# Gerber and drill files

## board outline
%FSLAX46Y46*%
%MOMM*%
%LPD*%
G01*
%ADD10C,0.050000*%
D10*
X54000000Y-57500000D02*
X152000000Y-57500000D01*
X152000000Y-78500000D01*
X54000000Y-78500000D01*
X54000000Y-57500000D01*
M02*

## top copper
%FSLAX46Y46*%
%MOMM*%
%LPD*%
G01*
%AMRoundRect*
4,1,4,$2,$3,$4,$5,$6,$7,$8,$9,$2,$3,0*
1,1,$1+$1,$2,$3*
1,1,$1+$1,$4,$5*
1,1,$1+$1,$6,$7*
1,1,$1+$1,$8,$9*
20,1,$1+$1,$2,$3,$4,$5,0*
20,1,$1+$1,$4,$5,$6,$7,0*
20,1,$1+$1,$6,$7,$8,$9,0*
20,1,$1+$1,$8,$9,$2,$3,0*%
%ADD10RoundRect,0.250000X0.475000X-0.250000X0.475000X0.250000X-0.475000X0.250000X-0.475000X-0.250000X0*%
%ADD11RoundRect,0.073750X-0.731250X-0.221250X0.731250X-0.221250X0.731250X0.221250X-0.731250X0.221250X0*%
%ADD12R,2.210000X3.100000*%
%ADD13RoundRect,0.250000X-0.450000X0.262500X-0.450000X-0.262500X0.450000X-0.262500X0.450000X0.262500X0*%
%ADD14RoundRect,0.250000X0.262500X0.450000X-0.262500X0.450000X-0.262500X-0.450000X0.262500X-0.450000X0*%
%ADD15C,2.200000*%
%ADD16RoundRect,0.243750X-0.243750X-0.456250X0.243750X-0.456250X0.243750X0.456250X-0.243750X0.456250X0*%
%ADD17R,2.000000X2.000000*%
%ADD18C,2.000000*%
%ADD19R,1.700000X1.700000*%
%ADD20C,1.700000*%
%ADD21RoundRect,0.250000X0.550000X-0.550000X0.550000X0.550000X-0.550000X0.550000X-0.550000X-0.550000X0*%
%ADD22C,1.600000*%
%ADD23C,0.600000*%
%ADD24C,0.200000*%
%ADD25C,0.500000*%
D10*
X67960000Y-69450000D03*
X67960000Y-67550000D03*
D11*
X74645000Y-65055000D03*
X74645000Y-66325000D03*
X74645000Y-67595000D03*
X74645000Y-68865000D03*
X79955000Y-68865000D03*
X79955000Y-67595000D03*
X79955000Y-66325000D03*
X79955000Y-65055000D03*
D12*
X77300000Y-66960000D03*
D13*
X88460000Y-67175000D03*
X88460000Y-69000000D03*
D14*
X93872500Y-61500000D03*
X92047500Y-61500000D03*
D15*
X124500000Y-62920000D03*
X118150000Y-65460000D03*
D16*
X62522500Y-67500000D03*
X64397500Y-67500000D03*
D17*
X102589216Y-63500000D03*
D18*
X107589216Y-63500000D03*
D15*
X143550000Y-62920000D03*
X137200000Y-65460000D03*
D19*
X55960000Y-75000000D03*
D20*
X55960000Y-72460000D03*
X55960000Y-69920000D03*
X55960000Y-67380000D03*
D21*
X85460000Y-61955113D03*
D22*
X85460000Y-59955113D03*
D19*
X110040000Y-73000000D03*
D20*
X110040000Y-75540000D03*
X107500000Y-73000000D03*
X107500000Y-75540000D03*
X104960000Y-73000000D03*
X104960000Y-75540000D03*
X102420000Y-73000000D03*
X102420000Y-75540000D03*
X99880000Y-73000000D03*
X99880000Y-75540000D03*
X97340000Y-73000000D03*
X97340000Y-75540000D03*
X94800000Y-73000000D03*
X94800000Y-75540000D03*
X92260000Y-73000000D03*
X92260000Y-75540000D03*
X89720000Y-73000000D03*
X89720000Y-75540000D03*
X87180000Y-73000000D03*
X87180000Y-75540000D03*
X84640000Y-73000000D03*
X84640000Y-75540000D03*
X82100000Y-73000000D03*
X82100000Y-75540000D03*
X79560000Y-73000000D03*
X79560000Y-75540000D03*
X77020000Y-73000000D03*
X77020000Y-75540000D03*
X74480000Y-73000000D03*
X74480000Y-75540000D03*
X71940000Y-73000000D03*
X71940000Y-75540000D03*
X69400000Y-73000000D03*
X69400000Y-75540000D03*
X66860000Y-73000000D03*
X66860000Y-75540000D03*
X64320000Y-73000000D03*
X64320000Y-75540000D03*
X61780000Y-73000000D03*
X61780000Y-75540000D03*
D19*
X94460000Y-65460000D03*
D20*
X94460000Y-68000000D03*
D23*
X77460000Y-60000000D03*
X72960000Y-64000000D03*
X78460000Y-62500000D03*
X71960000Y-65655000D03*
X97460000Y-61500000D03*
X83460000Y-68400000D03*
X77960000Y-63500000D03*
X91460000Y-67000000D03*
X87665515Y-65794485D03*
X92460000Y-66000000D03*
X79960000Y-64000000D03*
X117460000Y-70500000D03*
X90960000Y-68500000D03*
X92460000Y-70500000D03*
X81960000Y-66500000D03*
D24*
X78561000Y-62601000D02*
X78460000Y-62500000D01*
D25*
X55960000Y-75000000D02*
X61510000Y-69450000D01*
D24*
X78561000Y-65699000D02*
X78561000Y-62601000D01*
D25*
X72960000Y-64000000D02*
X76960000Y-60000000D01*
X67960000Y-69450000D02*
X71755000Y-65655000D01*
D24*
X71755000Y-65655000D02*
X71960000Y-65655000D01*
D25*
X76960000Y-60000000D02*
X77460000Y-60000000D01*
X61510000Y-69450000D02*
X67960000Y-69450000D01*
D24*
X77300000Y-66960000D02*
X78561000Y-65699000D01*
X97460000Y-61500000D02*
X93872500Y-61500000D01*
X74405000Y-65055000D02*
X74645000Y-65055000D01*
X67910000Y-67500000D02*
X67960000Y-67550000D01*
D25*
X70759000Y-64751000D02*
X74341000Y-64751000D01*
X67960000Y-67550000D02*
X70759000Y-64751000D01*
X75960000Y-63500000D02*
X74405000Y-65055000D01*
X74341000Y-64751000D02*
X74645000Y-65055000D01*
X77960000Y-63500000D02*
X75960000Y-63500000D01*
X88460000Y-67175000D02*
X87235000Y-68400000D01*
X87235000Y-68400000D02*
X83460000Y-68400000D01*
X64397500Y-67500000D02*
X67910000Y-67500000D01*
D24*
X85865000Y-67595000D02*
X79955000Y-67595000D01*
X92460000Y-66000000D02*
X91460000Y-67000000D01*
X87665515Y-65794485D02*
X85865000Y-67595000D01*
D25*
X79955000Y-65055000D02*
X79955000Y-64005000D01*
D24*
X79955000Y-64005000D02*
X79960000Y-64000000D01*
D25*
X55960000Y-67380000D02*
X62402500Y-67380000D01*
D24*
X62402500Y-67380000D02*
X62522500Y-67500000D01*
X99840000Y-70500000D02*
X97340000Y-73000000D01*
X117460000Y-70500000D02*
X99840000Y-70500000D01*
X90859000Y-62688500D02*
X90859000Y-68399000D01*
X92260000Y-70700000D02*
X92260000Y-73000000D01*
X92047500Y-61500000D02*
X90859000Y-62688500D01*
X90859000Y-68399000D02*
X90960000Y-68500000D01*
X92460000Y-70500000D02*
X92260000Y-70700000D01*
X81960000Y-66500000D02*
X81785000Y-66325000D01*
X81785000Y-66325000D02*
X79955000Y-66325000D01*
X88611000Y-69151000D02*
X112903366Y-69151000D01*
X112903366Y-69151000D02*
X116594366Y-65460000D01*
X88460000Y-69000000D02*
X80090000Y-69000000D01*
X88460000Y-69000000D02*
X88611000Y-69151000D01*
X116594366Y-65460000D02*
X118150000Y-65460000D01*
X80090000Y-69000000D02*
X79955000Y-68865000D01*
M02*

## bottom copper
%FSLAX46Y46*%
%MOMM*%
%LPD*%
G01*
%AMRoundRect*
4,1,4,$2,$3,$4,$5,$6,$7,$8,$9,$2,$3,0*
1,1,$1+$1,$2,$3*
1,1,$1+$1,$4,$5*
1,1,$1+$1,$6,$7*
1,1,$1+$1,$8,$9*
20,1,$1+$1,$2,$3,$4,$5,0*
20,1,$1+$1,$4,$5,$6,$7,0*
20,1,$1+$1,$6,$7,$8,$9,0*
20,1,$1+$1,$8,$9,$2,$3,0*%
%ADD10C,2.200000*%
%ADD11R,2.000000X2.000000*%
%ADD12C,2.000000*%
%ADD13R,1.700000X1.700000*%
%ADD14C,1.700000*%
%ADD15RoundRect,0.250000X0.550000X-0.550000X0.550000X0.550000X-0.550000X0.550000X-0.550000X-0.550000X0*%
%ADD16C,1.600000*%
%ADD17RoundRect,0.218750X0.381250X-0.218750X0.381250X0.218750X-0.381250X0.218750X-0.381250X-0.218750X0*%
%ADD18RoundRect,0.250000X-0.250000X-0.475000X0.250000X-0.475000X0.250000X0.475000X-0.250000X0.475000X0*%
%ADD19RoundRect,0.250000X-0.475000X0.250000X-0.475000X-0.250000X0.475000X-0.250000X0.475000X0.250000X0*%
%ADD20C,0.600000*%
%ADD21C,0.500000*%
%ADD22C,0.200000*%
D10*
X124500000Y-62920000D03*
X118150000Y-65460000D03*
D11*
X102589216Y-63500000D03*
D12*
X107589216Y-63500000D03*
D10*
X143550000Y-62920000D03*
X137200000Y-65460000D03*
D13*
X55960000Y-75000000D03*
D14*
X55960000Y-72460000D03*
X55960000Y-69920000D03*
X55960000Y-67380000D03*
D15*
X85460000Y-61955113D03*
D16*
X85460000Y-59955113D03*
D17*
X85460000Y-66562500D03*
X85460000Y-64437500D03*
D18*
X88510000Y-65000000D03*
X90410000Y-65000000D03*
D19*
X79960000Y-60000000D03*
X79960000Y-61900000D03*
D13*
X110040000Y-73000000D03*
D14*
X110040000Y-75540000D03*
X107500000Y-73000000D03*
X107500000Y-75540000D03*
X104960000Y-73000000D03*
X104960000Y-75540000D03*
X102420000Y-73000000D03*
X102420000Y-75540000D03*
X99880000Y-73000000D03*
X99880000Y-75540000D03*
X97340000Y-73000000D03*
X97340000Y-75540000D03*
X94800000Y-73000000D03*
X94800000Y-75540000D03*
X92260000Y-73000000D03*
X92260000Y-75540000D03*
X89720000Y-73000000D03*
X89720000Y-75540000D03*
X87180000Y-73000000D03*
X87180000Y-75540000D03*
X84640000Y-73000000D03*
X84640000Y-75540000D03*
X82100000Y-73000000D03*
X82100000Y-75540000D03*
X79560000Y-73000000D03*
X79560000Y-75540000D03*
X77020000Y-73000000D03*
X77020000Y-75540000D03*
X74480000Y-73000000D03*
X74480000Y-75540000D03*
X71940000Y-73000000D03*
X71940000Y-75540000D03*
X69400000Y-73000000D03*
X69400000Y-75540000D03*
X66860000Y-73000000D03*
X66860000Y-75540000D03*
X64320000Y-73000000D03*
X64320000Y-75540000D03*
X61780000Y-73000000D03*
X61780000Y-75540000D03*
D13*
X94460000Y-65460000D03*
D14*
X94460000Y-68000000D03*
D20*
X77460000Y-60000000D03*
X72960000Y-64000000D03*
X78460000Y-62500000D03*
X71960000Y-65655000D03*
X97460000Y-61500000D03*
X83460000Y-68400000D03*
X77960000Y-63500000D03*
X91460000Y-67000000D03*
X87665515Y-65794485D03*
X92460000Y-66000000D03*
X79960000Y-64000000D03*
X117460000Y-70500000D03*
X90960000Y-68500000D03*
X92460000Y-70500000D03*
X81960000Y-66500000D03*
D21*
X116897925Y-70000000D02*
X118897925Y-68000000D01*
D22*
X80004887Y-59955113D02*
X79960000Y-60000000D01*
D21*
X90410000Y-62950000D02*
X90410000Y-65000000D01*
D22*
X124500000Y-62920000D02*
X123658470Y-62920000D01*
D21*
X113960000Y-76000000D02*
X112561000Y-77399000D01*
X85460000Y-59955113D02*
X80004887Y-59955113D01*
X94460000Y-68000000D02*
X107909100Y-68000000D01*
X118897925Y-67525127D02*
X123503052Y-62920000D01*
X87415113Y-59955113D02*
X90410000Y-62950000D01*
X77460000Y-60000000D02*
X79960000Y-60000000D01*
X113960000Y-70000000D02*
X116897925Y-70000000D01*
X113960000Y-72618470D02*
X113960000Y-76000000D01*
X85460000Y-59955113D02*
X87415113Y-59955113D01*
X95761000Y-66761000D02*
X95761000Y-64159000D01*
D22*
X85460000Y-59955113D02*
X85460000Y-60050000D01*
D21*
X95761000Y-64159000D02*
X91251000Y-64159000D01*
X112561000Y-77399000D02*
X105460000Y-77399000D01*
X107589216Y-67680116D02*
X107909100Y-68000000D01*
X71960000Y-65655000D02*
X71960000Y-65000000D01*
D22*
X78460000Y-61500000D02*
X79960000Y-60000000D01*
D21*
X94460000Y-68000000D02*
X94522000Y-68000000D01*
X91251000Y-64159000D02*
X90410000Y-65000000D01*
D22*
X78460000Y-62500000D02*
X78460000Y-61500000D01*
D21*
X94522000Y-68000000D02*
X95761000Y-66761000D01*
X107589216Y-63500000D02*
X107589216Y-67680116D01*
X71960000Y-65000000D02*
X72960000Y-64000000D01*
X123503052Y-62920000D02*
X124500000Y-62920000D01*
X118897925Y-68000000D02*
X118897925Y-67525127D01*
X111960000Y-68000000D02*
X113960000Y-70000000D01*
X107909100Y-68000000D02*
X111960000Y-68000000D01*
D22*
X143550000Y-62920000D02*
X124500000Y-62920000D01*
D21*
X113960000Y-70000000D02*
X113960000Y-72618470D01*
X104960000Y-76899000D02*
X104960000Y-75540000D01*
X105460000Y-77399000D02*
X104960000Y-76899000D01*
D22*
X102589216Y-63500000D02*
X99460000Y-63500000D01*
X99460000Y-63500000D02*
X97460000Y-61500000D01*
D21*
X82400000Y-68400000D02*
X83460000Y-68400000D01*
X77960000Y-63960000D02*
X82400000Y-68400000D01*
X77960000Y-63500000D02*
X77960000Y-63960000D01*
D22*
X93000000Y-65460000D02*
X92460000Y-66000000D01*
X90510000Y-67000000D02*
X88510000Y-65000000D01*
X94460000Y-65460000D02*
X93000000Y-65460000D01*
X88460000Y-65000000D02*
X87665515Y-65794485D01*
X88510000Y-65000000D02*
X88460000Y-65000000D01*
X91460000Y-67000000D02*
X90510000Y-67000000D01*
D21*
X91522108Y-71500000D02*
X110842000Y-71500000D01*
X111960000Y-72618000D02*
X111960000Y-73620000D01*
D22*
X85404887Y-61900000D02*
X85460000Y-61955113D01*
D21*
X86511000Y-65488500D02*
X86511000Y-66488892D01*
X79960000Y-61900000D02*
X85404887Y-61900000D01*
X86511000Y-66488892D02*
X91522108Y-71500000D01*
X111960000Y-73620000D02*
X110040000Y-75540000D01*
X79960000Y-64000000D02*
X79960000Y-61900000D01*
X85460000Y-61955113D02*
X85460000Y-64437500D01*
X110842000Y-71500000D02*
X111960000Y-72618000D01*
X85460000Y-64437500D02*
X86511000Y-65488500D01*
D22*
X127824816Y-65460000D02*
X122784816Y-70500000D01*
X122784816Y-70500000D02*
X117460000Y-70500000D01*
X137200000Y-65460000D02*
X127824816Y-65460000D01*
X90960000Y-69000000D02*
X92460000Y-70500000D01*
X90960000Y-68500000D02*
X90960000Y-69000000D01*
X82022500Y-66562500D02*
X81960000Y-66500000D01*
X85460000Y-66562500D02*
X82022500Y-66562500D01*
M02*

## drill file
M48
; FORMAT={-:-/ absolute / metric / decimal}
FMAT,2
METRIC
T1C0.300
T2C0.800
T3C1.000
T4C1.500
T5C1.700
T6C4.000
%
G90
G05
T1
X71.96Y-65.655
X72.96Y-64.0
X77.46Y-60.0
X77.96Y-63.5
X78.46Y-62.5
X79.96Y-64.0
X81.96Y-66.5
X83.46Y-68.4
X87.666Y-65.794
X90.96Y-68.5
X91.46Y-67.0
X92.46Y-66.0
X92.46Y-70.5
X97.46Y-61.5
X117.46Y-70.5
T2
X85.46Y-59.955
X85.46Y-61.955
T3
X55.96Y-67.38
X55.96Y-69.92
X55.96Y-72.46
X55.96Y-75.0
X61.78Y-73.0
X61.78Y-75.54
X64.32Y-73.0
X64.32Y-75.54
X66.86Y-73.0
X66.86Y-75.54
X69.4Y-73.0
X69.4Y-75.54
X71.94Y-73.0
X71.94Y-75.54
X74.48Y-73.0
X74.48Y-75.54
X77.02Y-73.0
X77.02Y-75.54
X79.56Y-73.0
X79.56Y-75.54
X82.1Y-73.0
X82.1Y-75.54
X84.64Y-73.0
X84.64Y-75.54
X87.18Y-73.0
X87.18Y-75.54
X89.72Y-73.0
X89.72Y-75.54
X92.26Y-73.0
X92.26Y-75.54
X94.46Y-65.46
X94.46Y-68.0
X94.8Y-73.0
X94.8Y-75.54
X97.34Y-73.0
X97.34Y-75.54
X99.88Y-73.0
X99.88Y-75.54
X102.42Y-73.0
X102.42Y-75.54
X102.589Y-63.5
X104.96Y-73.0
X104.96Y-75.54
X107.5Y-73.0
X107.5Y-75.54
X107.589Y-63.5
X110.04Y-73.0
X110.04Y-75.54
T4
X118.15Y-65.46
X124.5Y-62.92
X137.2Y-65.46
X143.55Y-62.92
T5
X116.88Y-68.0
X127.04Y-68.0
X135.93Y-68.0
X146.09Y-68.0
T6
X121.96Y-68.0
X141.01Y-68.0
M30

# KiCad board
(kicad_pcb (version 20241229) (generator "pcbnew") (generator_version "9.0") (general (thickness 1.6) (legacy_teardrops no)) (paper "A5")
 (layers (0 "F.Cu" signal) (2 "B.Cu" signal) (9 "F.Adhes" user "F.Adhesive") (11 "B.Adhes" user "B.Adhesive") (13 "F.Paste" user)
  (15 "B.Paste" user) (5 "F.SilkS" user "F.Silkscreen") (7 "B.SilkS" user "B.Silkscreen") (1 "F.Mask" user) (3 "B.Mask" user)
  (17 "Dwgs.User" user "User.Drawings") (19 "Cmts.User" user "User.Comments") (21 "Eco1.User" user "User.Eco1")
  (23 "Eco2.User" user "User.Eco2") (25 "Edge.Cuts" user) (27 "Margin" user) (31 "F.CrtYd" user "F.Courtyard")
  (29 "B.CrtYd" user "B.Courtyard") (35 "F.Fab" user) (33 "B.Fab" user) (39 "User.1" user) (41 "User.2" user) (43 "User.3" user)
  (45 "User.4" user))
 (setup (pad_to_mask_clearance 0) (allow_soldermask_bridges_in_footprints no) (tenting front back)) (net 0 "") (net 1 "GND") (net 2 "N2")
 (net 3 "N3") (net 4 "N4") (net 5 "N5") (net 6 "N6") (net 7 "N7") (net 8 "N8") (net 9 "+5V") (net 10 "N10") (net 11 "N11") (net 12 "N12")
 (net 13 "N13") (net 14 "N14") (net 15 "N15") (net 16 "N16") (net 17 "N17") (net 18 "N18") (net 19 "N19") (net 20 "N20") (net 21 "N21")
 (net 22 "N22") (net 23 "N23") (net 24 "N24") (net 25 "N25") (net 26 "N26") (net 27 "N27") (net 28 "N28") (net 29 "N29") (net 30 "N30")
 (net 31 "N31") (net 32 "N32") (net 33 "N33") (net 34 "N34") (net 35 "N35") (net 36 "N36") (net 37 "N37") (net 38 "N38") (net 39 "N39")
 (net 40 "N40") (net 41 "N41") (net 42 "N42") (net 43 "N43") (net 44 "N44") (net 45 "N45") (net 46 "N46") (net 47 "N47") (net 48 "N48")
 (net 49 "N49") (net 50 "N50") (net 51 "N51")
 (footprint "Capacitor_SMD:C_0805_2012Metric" (layer "F.Cu") (at 67.96 68.5 90)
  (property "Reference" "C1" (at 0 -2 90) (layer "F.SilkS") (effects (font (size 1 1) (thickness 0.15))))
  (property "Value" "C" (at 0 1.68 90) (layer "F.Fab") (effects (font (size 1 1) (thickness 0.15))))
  (pad "1" smd roundrect (at -0.95 0 90) (size 1 1.45) (layers "F.Cu" "F.Mask" "F.Paste") (roundrect_rratio 0.25) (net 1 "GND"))
  (pad "2" smd roundrect (at 0.95 0 90) (size 1 1.45) (layers "F.Cu" "F.Mask" "F.Paste") (roundrect_rratio 0.25) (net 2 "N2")))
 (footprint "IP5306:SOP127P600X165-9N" (layer "F.Cu") (at 77.3 66.96)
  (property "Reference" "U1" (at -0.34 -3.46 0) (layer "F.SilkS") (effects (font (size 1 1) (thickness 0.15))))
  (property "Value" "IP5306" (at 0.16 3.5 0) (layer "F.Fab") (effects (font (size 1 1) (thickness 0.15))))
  (pad "1" smd roundrect (at -2.655 -1.905) (size 1.61 0.59) (layers "F.Cu" "F.Mask" "F.Paste") (roundrect_rratio 0.125) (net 2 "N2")
   (solder_mask_margin 0.102))
  (pad "2" smd roundrect (at -2.655 -0.635) (size 1.61 0.59) (layers "F.Cu" "F.Mask" "F.Paste") (roundrect_rratio 0.125) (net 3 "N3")
   (solder_mask_margin 0.102))
  (pad "3" smd roundrect (at -2.655 0.635) (size 1.61 0.59) (layers "F.Cu" "F.Mask" "F.Paste") (roundrect_rratio 0.125) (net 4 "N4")
   (solder_mask_margin 0.102))
  (pad "4" smd roundrect (at -2.655 1.905) (size 1.61 0.59) (layers "F.Cu" "F.Mask" "F.Paste") (roundrect_rratio 0.125) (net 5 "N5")
   (solder_mask_margin 0.102))
  (pad "5" smd roundrect (at 2.655 1.905) (size 1.61 0.59) (layers "F.Cu" "F.Mask" "F.Paste") (roundrect_rratio 0.125) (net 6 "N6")
   (solder_mask_margin 0.102))
  (pad "6" smd roundrect (at 2.655 0.635) (size 1.61 0.59) (layers "F.Cu" "F.Mask" "F.Paste") (roundrect_rratio 0.125) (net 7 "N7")
   (solder_mask_margin 0.102))
  (pad "7" smd roundrect (at 2.655 -0.635) (size 1.61 0.59) (layers "F.Cu" "F.Mask" "F.Paste") (roundrect_rratio 0.125) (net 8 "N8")
   (solder_mask_margin 0.102))
  (pad "8" smd roundrect (at 2.655 -1.905) (size 1.61 0.59) (layers "F.Cu" "F.Mask" "F.Paste") (roundrect_rratio 0.125) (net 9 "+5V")
   (solder_mask_margin 0.102))
  (pad "9" smd rect (at 0 0) (size 2.21 3.1) (layers "F.Cu" "F.Mask") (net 1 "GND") (solder_mask_margin 0.102)))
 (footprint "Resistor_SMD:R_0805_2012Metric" (layer "F.Cu") (at 88.46 68.0875 -90)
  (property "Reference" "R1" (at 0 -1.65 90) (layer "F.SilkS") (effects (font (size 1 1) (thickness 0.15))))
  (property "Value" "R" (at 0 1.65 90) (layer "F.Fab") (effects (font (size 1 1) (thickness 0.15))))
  (pad "1" smd roundrect (at -0.9125 0 270) (size 1.025 1.4) (layers "F.Cu" "F.Mask" "F.Paste") (roundrect_rratio 0.243902) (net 2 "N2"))
  (pad "2" smd roundrect (at 0.9125 0 270) (size 1.025 1.4) (layers "F.Cu" "F.Mask" "F.Paste") (roundrect_rratio 0.243902) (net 6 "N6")))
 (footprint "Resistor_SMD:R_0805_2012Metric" (layer "F.Cu") (at 92.96 61.5 180)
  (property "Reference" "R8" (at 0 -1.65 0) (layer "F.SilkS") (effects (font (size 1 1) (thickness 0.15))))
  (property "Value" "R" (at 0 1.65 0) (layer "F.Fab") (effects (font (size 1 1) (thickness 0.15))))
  (pad "1" smd roundrect (at -0.9125 0 180) (size 1.025 1.4) (layers "F.Cu" "F.Mask" "F.Paste") (roundrect_rratio 0.243902) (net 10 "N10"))
  (pad "2" smd roundrect (at 0.9125 0 180) (size 1.025 1.4) (layers "F.Cu" "F.Mask" "F.Paste") (roundrect_rratio 0.243902) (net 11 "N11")))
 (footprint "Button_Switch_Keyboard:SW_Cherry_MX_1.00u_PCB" (layer "F.Cu") (at 124.5 62.92)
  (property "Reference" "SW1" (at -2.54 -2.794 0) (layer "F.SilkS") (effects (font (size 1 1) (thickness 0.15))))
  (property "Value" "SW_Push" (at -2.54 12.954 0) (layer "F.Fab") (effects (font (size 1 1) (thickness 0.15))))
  (pad "" np_thru_hole circle (at -7.62 5.08) (size 1.7 1.7) (drill 1.7) (layers "*.Cu" "*.Mask"))
  (pad "" np_thru_hole circle (at -2.54 5.08) (size 4 4) (drill 4) (layers "*.Cu" "*.Mask"))
  (pad "" np_thru_hole circle (at 2.54 5.08) (size 1.7 1.7) (drill 1.7) (layers "*.Cu" "*.Mask"))
  (pad "1" thru_hole circle (at 0 0) (size 2.2 2.2) (drill 1.5) (layers "*.Cu" "*.Mask") (remove_unused_layers no) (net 1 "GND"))
  (pad "2" thru_hole circle (at -6.35 2.54) (size 2.2 2.2) (drill 1.5) (layers "*.Cu" "*.Mask") (remove_unused_layers no) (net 6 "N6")))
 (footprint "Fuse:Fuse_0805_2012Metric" (layer "F.Cu") (at 63.46 67.5)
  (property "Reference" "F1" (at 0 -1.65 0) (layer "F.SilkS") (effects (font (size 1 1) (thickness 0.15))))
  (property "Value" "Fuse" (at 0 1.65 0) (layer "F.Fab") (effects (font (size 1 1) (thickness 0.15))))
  (pad "1" smd roundrect (at -0.9375 0) (size 0.975 1.4) (layers "F.Cu" "F.Mask" "F.Paste") (roundrect_rratio 0.25) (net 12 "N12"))
  (pad "2" smd roundrect (at 0.9375 0) (size 0.975 1.4) (layers "F.Cu" "F.Mask" "F.Paste") (roundrect_rratio 0.25) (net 2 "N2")))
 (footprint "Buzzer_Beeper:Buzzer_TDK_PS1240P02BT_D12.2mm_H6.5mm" (layer "F.Cu") (at 102.589216 63.5)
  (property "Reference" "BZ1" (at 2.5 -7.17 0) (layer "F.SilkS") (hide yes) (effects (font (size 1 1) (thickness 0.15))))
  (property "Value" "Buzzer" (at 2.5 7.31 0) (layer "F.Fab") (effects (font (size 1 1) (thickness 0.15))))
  (pad "1" thru_hole rect (at 0 0) (size 2 2) (drill 1) (layers "*.Cu" "*.Mask") (remove_unused_layers no) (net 10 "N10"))
  (pad "2" thru_hole circle (at 5 0) (size 2 2) (drill 1) (layers "*.Cu" "*.Mask") (remove_unused_layers no) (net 1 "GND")))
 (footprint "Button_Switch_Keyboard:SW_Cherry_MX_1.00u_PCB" (layer "F.Cu") (at 143.55 62.92)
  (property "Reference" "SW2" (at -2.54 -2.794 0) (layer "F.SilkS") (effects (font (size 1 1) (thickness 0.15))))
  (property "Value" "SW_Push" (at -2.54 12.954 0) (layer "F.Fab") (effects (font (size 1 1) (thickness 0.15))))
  (pad "" np_thru_hole circle (at -7.62 5.08) (size 1.7 1.7) (drill 1.7) (layers "*.Cu" "*.Mask"))
  (pad "" np_thru_hole circle (at -2.54 5.08) (size 4 4) (drill 4) (layers "*.Cu" "*.Mask"))
  (pad "" np_thru_hole circle (at 2.54 5.08) (size 1.7 1.7) (drill 1.7) (layers "*.Cu" "*.Mask"))
  (pad "1" thru_hole circle (at 0 0) (size 2.2 2.2) (drill 1.5) (layers "*.Cu" "*.Mask") (remove_unused_layers no) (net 1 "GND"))
  (pad "2" thru_hole circle (at -6.35 2.54) (size 2.2 2.2) (drill 1.5) (layers "*.Cu" "*.Mask") (remove_unused_layers no) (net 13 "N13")))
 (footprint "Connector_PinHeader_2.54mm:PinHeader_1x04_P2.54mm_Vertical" (layer "F.Cu") (at 55.96 75 180)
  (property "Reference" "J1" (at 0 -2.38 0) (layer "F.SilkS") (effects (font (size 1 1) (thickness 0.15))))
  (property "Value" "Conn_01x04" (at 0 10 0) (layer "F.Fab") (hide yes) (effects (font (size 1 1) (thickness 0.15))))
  (pad "1" thru_hole rect (at 0 0 180) (size 1.7 1.7) (drill 1) (layers "*.Cu" "*.Mask") (remove_unused_layers no) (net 1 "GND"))
  (pad "2" thru_hole circle (at 0 2.54 180) (size 1.7 1.7) (drill 1) (layers "*.Cu" "*.Mask") (remove_unused_layers no) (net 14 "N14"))
  (pad "3" thru_hole circle (at 0 5.08 180) (size 1.7 1.7) (drill 1) (layers "*.Cu" "*.Mask") (remove_unused_layers no) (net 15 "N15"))
  (pad "4" thru_hole circle (at 0 7.62 180) (size 1.7 1.7) (drill 1) (layers "*.Cu" "*.Mask") (remove_unused_layers no) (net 12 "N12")))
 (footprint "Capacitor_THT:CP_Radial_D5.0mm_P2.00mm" (layer "B.Cu") (at 85.46 61.955113 90)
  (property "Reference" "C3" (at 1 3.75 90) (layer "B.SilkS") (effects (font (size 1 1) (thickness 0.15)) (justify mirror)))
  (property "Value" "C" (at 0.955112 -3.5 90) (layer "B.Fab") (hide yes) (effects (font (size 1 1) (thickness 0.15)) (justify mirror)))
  (pad "1" thru_hole roundrect (at 0 0 90) (size 1.6 1.6) (drill 0.8) (layers "*.Cu" "*.Mask") (remove_unused_layers no)
   (roundrect_rratio 0.15625) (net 9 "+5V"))
  (pad "2" thru_hole circle (at 2 0 90) (size 1.6 1.6) (drill 0.8) (layers "*.Cu" "*.Mask") (remove_unused_layers no) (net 1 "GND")))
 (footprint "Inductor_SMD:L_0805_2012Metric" (layer "B.Cu") (at 85.46 65.5 90)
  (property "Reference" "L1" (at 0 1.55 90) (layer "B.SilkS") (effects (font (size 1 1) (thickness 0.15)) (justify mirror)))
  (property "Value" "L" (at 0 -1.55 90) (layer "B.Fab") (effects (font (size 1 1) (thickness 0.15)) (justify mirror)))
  (pad "1" smd roundrect (at -1.0625 0 90) (size 0.875 1.2) (layers "B.Cu" "B.Mask" "B.Paste") (roundrect_rratio 0.25) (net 8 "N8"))
  (pad "2" smd roundrect (at 1.0625 0 90) (size 0.875 1.2) (layers "B.Cu" "B.Mask" "B.Paste") (roundrect_rratio 0.25) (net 9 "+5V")))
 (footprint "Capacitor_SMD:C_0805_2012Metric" (layer "B.Cu") (at 89.46 65)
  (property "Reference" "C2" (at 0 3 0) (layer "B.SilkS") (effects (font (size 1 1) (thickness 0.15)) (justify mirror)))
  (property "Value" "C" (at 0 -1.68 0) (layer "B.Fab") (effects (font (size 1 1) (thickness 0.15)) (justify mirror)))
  (pad "1" smd roundrect (at -0.95 0) (size 1 1.45) (layers "B.Cu" "B.Mask" "B.Paste") (roundrect_rratio 0.25) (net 7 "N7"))
  (pad "2" smd roundrect (at 0.95 0) (size 1 1.45) (layers "B.Cu" "B.Mask" "B.Paste") (roundrect_rratio 0.25) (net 1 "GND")))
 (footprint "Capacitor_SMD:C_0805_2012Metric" (layer "B.Cu") (at 79.96 60.95 -90)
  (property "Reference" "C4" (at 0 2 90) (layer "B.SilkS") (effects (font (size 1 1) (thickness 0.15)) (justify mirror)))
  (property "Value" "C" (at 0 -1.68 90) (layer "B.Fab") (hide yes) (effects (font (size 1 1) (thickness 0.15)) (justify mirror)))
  (pad "1" smd roundrect (at -0.95 0 270) (size 1 1.45) (layers "B.Cu" "B.Mask" "B.Paste") (roundrect_rratio 0.25) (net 1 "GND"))
  (pad "2" smd roundrect (at 0.95 0 270) (size 1 1.45) (layers "B.Cu" "B.Mask" "B.Paste") (roundrect_rratio 0.25) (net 9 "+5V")))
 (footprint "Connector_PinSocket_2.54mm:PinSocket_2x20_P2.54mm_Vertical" (layer "B.Cu") (at 110.04 73 90)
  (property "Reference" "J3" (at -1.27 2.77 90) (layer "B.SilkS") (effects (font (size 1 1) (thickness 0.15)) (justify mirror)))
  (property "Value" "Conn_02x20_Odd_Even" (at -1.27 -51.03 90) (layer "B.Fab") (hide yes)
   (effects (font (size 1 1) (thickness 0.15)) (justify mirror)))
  (pad "1" thru_hole rect (at 0 0 90) (size 1.7 1.7) (drill 1) (layers "*.Cu" "*.Mask") (remove_unused_layers no) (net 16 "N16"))
  (pad "2" thru_hole circle (at -2.54 0 90) (size 1.7 1.7) (drill 1) (layers "*.Cu" "*.Mask") (remove_unused_layers no) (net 9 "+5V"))
  (pad "3" thru_hole circle (at 0 -2.54 90) (size 1.7 1.7) (drill 1) (layers "*.Cu" "*.Mask") (remove_unused_layers no) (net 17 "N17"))
  (pad "4" thru_hole circle (at -2.54 -2.54 90) (size 1.7 1.7) (drill 1) (layers "*.Cu" "*.Mask") (remove_unused_layers no) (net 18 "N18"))
  (pad "5" thru_hole circle (at 0 -5.08 90) (size 1.7 1.7) (drill 1) (layers "*.Cu" "*.Mask") (remove_unused_layers no) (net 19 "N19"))
  (pad "6" thru_hole circle (at -2.54 -5.08 90) (size 1.7 1.7) (drill 1) (layers "*.Cu" "*.Mask") (remove_unused_layers no) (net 1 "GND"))
  (pad "7" thru_hole circle (at 0 -7.62 90) (size 1.7 1.7) (drill 1) (layers "*.Cu" "*.Mask") (remove_unused_layers no) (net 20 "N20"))
  (pad "8" thru_hole circle (at -2.54 -7.62 90) (size 1.7 1.7) (drill 1) (layers "*.Cu" "*.Mask") (remove_unused_layers no) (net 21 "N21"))
  (pad "9" thru_hole circle (at 0 -10.16 90) (size 1.7 1.7) (drill 1) (layers "*.Cu" "*.Mask") (remove_unused_layers no) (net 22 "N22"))
  (pad "10" thru_hole circle (at -2.54 -10.16 90) (size 1.7 1.7) (drill 1) (layers "*.Cu" "*.Mask") (remove_unused_layers no) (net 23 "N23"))
  (pad "11" thru_hole circle (at 0 -12.7 90) (size 1.7 1.7) (drill 1) (layers "*.Cu" "*.Mask") (remove_unused_layers no) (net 13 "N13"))
  (pad "12" thru_hole circle (at -2.54 -12.7 90) (size 1.7 1.7) (drill 1) (layers "*.Cu" "*.Mask") (remove_unused_layers no) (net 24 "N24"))
  (pad "13" thru_hole circle (at 0 -15.24 90) (size 1.7 1.7) (drill 1) (layers "*.Cu" "*.Mask") (remove_unused_layers no) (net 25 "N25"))
  (pad "14" thru_hole circle (at -2.54 -15.24 90) (size 1.7 1.7) (drill 1) (layers "*.Cu" "*.Mask") (remove_unused_layers no) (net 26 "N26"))
  (pad "15" thru_hole circle (at 0 -17.78 90) (size 1.7 1.7) (drill 1) (layers "*.Cu" "*.Mask") (remove_unused_layers no) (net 11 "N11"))
  (pad "16" thru_hole circle (at -2.54 -17.78 90) (size 1.7 1.7) (drill 1) (layers "*.Cu" "*.Mask") (remove_unused_layers no) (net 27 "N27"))
  (pad "17" thru_hole circle (at 0 -20.32 90) (size 1.7 1.7) (drill 1) (layers "*.Cu" "*.Mask") (remove_unused_layers no) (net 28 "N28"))
  (pad "18" thru_hole circle (at -2.54 -20.32 90) (size 1.7 1.7) (drill 1) (layers "*.Cu" "*.Mask") (remove_unused_layers no) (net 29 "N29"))
  (pad "19" thru_hole circle (at 0 -22.86 90) (size 1.7 1.7) (drill 1) (layers "*.Cu" "*.Mask") (remove_unused_layers no) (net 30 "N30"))
  (pad "20" thru_hole circle (at -2.54 -22.86 90) (size 1.7 1.7) (drill 1) (layers "*.Cu" "*.Mask") (remove_unused_layers no) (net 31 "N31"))
  (pad "21" thru_hole circle (at 0 -25.4 90) (size 1.7 1.7) (drill 1) (layers "*.Cu" "*.Mask") (remove_unused_layers no) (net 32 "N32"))
  (pad "22" thru_hole circle (at -2.54 -25.4 90) (size 1.7 1.7) (drill 1) (layers "*.Cu" "*.Mask") (remove_unused_layers no) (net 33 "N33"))
  (pad "23" thru_hole circle (at 0 -27.94 90) (size 1.7 1.7) (drill 1) (layers "*.Cu" "*.Mask") (remove_unused_layers no) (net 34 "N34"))
  (pad "24" thru_hole circle (at -2.54 -27.94 90) (size 1.7 1.7) (drill 1) (layers "*.Cu" "*.Mask") (remove_unused_layers no) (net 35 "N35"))
  (pad "25" thru_hole circle (at 0 -30.48 90) (size 1.7 1.7) (drill 1) (layers "*.Cu" "*.Mask") (remove_unused_layers no) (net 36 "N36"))
  (pad "26" thru_hole circle (at -2.54 -30.48 90) (size 1.7 1.7) (drill 1) (layers "*.Cu" "*.Mask") (remove_unused_layers no) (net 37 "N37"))
  (pad "27" thru_hole circle (at 0 -33.02 90) (size 1.7 1.7) (drill 1) (layers "*.Cu" "*.Mask") (remove_unused_layers no) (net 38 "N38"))
  (pad "28" thru_hole circle (at -2.54 -33.02 90) (size 1.7 1.7) (drill 1) (layers "*.Cu" "*.Mask") (remove_unused_layers no) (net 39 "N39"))
  (pad "29" thru_hole circle (at 0 -35.56 90) (size 1.7 1.7) (drill 1) (layers "*.Cu" "*.Mask") (remove_unused_layers no) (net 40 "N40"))
  (pad "30" thru_hole circle (at -2.54 -35.56 90) (size 1.7 1.7) (drill 1) (layers "*.Cu" "*.Mask") (remove_unused_layers no) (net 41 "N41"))
  (pad "31" thru_hole circle (at 0 -38.1 90) (size 1.7 1.7) (drill 1) (layers "*.Cu" "*.Mask") (remove_unused_layers no) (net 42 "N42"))
  (pad "32" thru_hole circle (at -2.54 -38.1 90) (size 1.7 1.7) (drill 1) (layers "*.Cu" "*.Mask") (remove_unused_layers no) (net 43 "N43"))
  (pad "33" thru_hole circle (at 0 -40.64 90) (size 1.7 1.7) (drill 1) (layers "*.Cu" "*.Mask") (remove_unused_layers no) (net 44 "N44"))
  (pad "34" thru_hole circle (at -2.54 -40.64 90) (size 1.7 1.7) (drill 1) (layers "*.Cu" "*.Mask") (remove_unused_layers no) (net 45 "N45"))
  (pad "35" thru_hole circle (at 0 -43.18 90) (size 1.7 1.7) (drill 1) (layers "*.Cu" "*.Mask") (remove_unused_layers no) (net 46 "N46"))
  (pad "36" thru_hole circle (at -2.54 -43.18 90) (size 1.7 1.7) (drill 1) (layers "*.Cu" "*.Mask") (remove_unused_layers no) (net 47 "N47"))
  (pad "37" thru_hole circle (at 0 -45.72 90) (size 1.7 1.7) (drill 1) (layers "*.Cu" "*.Mask") (remove_unused_layers no) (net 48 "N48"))
  (pad "38" thru_hole circle (at -2.54 -45.72 90) (size 1.7 1.7) (drill 1) (layers "*.Cu" "*.Mask") (remove_unused_layers no) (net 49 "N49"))
  (pad "39" thru_hole circle (at 0 -48.26 90) (size 1.7 1.7) (drill 1) (layers "*.Cu" "*.Mask") (remove_unused_layers no) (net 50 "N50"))
  (pad "40" thru_hole circle (at -2.54 -48.26 90) (size 1.7 1.7) (drill 1) (layers "*.Cu" "*.Mask") (remove_unused_layers no) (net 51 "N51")))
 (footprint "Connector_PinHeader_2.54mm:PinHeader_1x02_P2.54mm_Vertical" (layer "B.Cu") (at 94.46 65.46 180)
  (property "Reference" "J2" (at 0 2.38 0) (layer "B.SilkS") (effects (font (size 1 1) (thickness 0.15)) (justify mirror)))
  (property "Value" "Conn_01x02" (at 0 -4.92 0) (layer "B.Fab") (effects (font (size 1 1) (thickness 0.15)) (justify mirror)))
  (pad "1" thru_hole rect (at 0 0 180) (size 1.7 1.7) (drill 1) (layers "*.Cu" "*.Mask") (remove_unused_layers no) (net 7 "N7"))
  (pad "2" thru_hole circle (at 0 -2.54 180) (size 1.7 1.7) (drill 1) (layers "*.Cu" "*.Mask") (remove_unused_layers no) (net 1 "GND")))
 (gr_rect (start 54 57.5) (end 152 78.5) (stroke (width 0.05) (type default)) (fill no) (layer "Edge.Cuts"))
 (segment (start 78.561 62.601) (end 78.46 62.5) (width 0.2) (layer "F.Cu") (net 1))
 (segment (start 55.96 75) (end 61.51 69.45) (width 0.5) (layer "F.Cu") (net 1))
 (segment (start 78.561 65.699) (end 78.561 62.601) (width 0.2) (layer "F.Cu") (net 1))
 (segment (start 72.96 64) (end 76.96 60) (width 0.5) (layer "F.Cu") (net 1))
 (segment (start 67.96 69.45) (end 71.755 65.655) (width 0.5) (layer "F.Cu") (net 1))
 (segment (start 71.755 65.655) (end 71.96 65.655) (width 0.2) (layer "F.Cu") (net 1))
 (segment (start 76.96 60) (end 77.46 60) (width 0.5) (layer "F.Cu") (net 1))
 (segment (start 61.51 69.45) (end 67.96 69.45) (width 0.5) (layer "F.Cu") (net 1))
 (segment (start 77.3 66.96) (end 78.561 65.699) (width 0.2) (layer "F.Cu") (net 1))
 (via (at 77.46 60) (size 0.6) (drill 0.3) (layers "F.Cu" "B.Cu") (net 1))
 (via (at 72.96 64) (size 0.6) (drill 0.3) (layers "F.Cu" "B.Cu") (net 1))
 (via (at 78.46 62.5) (size 0.6) (drill 0.3) (layers "F.Cu" "B.Cu") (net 1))
 (via (at 71.96 65.655) (size 0.6) (drill 0.3) (layers "F.Cu" "B.Cu") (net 1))
 (segment (start 116.897925 70) (end 118.897925 68) (width 0.5) (layer "B.Cu") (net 1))
 (segment (start 80.004887 59.955113) (end 79.96 60) (width 0.2) (layer "B.Cu") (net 1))
 (segment (start 90.41 62.95) (end 90.41 65) (width 0.5) (layer "B.Cu") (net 1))
 (segment (start 124.5 62.92) (end 123.65847 62.92) (width 0.2) (layer "B.Cu") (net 1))
 (segment (start 113.96 76) (end 112.561 77.399) (width 0.5) (layer "B.Cu") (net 1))
 (segment (start 85.46 59.955113) (end 80.004887 59.955113) (width 0.5) (layer "B.Cu") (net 1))
 (segment (start 94.46 68) (end 107.9091 68) (width 0.5) (layer "B.Cu") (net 1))
 (segment (start 118.897925 67.525127) (end 123.503052 62.92) (width 0.5) (layer "B.Cu") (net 1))
 (segment (start 87.415113 59.955113) (end 90.41 62.95) (width 0.5) (layer "B.Cu") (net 1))
 (segment (start 77.46 60) (end 79.96 60) (width 0.5) (layer "B.Cu") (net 1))
 (segment (start 113.96 70) (end 116.897925 70) (width 0.5) (layer "B.Cu") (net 1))
 (segment (start 113.96 72.61847) (end 113.96 76) (width 0.5) (layer "B.Cu") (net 1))
 (segment (start 85.46 59.955113) (end 87.415113 59.955113) (width 0.5) (layer "B.Cu") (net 1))
 (segment (start 95.761 66.761) (end 95.761 64.159) (width 0.5) (layer "B.Cu") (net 1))
 (segment (start 85.46 59.955113) (end 85.46 60.05) (width 0.2) (layer "B.Cu") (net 1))
 (segment (start 95.761 64.159) (end 91.251 64.159) (width 0.5) (layer "B.Cu") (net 1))
 (segment (start 112.561 77.399) (end 105.46 77.399) (width 0.5) (layer "B.Cu") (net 1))
 (segment (start 107.589216 67.680116) (end 107.9091 68) (width 0.5) (layer "B.Cu") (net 1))
 (segment (start 71.96 65.655) (end 71.96 65) (width 0.5) (layer "B.Cu") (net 1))
 (segment (start 78.46 61.5) (end 79.96 60) (width 0.2) (layer "B.Cu") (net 1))
 (segment (start 94.46 68) (end 94.522 68) (width 0.5) (layer "B.Cu") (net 1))
 (segment (start 91.251 64.159) (end 90.41 65) (width 0.5) (layer "B.Cu") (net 1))
 (segment (start 78.46 62.5) (end 78.46 61.5) (width 0.2) (layer "B.Cu") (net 1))
 (segment (start 94.522 68) (end 95.761 66.761) (width 0.5) (layer "B.Cu") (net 1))
 (segment (start 107.589216 63.5) (end 107.589216 67.680116) (width 0.5) (layer "B.Cu") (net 1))
 (segment (start 71.96 65) (end 72.96 64) (width 0.5) (layer "B.Cu") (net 1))
 (segment (start 123.503052 62.92) (end 124.5 62.92) (width 0.5) (layer "B.Cu") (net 1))
 (segment (start 118.897925 68) (end 118.897925 67.525127) (width 0.5) (layer "B.Cu") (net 1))
 (segment (start 111.96 68) (end 113.96 70) (width 0.5) (layer "B.Cu") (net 1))
 (segment (start 107.9091 68) (end 111.96 68) (width 0.5) (layer "B.Cu") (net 1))
 (segment (start 143.55 62.92) (end 124.5 62.92) (width 0.2) (layer "B.Cu") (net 1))
 (segment (start 113.96 70) (end 113.96 72.61847) (width 0.5) (layer "B.Cu") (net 1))
 (segment (start 104.96 76.899) (end 104.96 75.54) (width 0.5) (layer "B.Cu") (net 1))
 (segment (start 105.46 77.399) (end 104.96 76.899) (width 0.5) (layer "B.Cu") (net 1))
 (segment (start 97.46 61.5) (end 93.8725 61.5) (width 0.2) (layer "F.Cu") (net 10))
 (via (at 97.46 61.5) (size 0.6) (drill 0.3) (layers "F.Cu" "B.Cu") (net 10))
 (segment (start 102.589216 63.5) (end 99.46 63.5) (width 0.2) (layer "B.Cu") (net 10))
 (segment (start 99.46 63.5) (end 97.46 61.5) (width 0.2) (layer "B.Cu") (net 10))
 (segment (start 74.405 65.055) (end 74.645 65.055) (width 0.2) (layer "F.Cu") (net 2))
 (segment (start 67.91 67.5) (end 67.96 67.55) (width 0.2) (layer "F.Cu") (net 2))
 (segment (start 70.759 64.751) (end 74.341 64.751) (width 0.5) (layer "F.Cu") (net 2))
 (segment (start 67.96 67.55) (end 70.759 64.751) (width 0.5) (layer "F.Cu") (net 2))
 (segment (start 75.96 63.5) (end 74.405 65.055) (width 0.5) (layer "F.Cu") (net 2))
 (segment (start 74.341 64.751) (end 74.645 65.055) (width 0.5) (layer "F.Cu") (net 2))
 (segment (start 77.96 63.5) (end 75.96 63.5) (width 0.5) (layer "F.Cu") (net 2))
 (segment (start 88.46 67.175) (end 87.235 68.4) (width 0.5) (layer "F.Cu") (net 2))
 (segment (start 87.235 68.4) (end 83.46 68.4) (width 0.5) (layer "F.Cu") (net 2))
 (segment (start 64.3975 67.5) (end 67.91 67.5) (width 0.5) (layer "F.Cu") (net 2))
 (via (at 83.46 68.4) (size 0.6) (drill 0.3) (layers "F.Cu" "B.Cu") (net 2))
 (via (at 77.96 63.5) (size 0.6) (drill 0.3) (layers "F.Cu" "B.Cu") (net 2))
 (segment (start 82.4 68.4) (end 83.46 68.4) (width 0.5) (layer "B.Cu") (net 2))
 (segment (start 77.96 63.96) (end 82.4 68.4) (width 0.5) (layer "B.Cu") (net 2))
 (segment (start 77.96 63.5) (end 77.96 63.96) (width 0.5) (layer "B.Cu") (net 2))
 (segment (start 85.865 67.595) (end 79.955 67.595) (width 0.2) (layer "F.Cu") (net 7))
 (segment (start 92.46 66) (end 91.46 67) (width 0.2) (layer "F.Cu") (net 7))
 (segment (start 87.665515 65.794485) (end 85.865 67.595) (width 0.2) (layer "F.Cu") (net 7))
 (via (at 91.46 67) (size 0.6) (drill 0.3) (layers "F.Cu" "B.Cu") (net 7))
 (via (at 87.665515 65.794485) (size 0.6) (drill 0.3) (layers "F.Cu" "B.Cu") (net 7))
 (via (at 92.46 66) (size 0.6) (drill 0.3) (layers "F.Cu" "B.Cu") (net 7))
 (segment (start 93 65.46) (end 92.46 66) (width 0.2) (layer "B.Cu") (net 7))
 (segment (start 90.51 67) (end 88.51 65) (width 0.2) (layer "B.Cu") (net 7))
 (segment (start 94.46 65.46) (end 93 65.46) (width 0.2) (layer "B.Cu") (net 7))
 (segment (start 88.46 65) (end 87.665515 65.794485) (width 0.2) (layer "B.Cu") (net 7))
 (segment (start 88.51 65) (end 88.46 65) (width 0.2) (layer "B.Cu") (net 7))
 (segment (start 91.46 67) (end 90.51 67) (width 0.2) (layer "B.Cu") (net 7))
 (segment (start 79.955 65.055) (end 79.955 64.005) (width 0.5) (layer "F.Cu") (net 9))
 (segment (start 79.955 64.005) (end 79.96 64) (width 0.2) (layer "F.Cu") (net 9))
 (via (at 79.96 64) (size 0.6) (drill 0.3) (layers "F.Cu" "B.Cu") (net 9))
 (segment (start 91.522108 71.5) (end 110.842 71.5) (width 0.5) (layer "B.Cu") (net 9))
 (segment (start 111.96 72.618) (end 111.96 73.62) (width 0.5) (layer "B.Cu") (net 9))
 (segment (start 85.404887 61.9) (end 85.46 61.955113) (width 0.2) (layer "B.Cu") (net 9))
 (segment (start 86.511 65.4885) (end 86.511 66.488892) (width 0.5) (layer "B.Cu") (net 9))
 (segment (start 79.96 61.9) (end 85.404887 61.9) (width 0.5) (layer "B.Cu") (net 9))
 (segment (start 86.511 66.488892) (end 91.522108 71.5) (width 0.5) (layer "B.Cu") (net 9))
 (segment (start 111.96 73.62) (end 110.04 75.54) (width 0.5) (layer "B.Cu") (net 9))
 (segment (start 79.96 64) (end 79.96 61.9) (width 0.5) (layer "B.Cu") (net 9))
 (segment (start 85.46 61.955113) (end 85.46 64.4375) (width 0.5) (layer "B.Cu") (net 9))
 (segment (start 110.842 71.5) (end 111.96 72.618) (width 0.5) (layer "B.Cu") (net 9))
 (segment (start 85.46 64.4375) (end 86.511 65.4885) (width 0.5) (layer "B.Cu") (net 9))
 (segment (start 55.96 67.38) (end 62.4025 67.38) (width 0.5) (layer "F.Cu") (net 12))
 (segment (start 62.4025 67.38) (end 62.5225 67.5) (width 0.2) (layer "F.Cu") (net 12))
 (segment (start 99.84 70.5) (end 97.34 73) (width 0.2) (layer "F.Cu") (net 13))
 (segment (start 117.46 70.5) (end 99.84 70.5) (width 0.2) (layer "F.Cu") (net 13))
 (via (at 117.46 70.5) (size 0.6) (drill 0.3) (layers "F.Cu" "B.Cu") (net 13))
 (segment (start 127.824816 65.46) (end 122.784816 70.5) (width 0.2) (layer "B.Cu") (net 13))
 (segment (start 122.784816 70.5) (end 117.46 70.5) (width 0.2) (layer "B.Cu") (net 13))
 (segment (start 137.2 65.46) (end 127.824816 65.46) (width 0.2) (layer "B.Cu") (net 13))
 (segment (start 90.859 62.6885) (end 90.859 68.399) (width 0.2) (layer "F.Cu") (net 11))
 (segment (start 92.26 70.7) (end 92.26 73) (width 0.2) (layer "F.Cu") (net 11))
 (segment (start 92.0475 61.5) (end 90.859 62.6885) (width 0.2) (layer "F.Cu") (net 11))
 (segment (start 90.859 68.399) (end 90.96 68.5) (width 0.2) (layer "F.Cu") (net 11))
 (segment (start 92.46 70.5) (end 92.26 70.7) (width 0.2) (layer "F.Cu") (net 11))
 (via (at 90.96 68.5) (size 0.6) (drill 0.3) (layers "F.Cu" "B.Cu") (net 11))
 (via (at 92.46 70.5) (size 0.6) (drill 0.3) (layers "F.Cu" "B.Cu") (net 11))
 (segment (start 90.96 69) (end 92.46 70.5) (width 0.2) (layer "B.Cu") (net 11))
 (segment (start 90.96 68.5) (end 90.96 69) (width 0.2) (layer "B.Cu") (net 11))
 (segment (start 81.96 66.5) (end 81.785 66.325) (width 0.2) (layer "F.Cu") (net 8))
 (segment (start 81.785 66.325) (end 79.955 66.325) (width 0.2) (layer "F.Cu") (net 8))
 (via (at 81.96 66.5) (size 0.6) (drill 0.3) (layers "F.Cu" "B.Cu") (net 8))
 (segment (start 82.0225 66.5625) (end 81.96 66.5) (width 0.2) (layer "B.Cu") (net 8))
 (segment (start 85.46 66.5625) (end 82.0225 66.5625) (width 0.2) (layer "B.Cu") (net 8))
 (segment (start 88.611 69.151) (end 112.903366 69.151) (width 0.2) (layer "F.Cu") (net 6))
 (segment (start 112.903366 69.151) (end 116.594366 65.46) (width 0.2) (layer "F.Cu") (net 6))
 (segment (start 88.46 69) (end 80.09 69) (width 0.2) (layer "F.Cu") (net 6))
 (segment (start 88.46 69) (end 88.611 69.151) (width 0.2) (layer "F.Cu") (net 6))
 (segment (start 116.594366 65.46) (end 118.15 65.46) (width 0.2) (layer "F.Cu") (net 6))
 (segment (start 80.09 69) (end 79.955 68.865) (width 0.2) (layer "F.Cu") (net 6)))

